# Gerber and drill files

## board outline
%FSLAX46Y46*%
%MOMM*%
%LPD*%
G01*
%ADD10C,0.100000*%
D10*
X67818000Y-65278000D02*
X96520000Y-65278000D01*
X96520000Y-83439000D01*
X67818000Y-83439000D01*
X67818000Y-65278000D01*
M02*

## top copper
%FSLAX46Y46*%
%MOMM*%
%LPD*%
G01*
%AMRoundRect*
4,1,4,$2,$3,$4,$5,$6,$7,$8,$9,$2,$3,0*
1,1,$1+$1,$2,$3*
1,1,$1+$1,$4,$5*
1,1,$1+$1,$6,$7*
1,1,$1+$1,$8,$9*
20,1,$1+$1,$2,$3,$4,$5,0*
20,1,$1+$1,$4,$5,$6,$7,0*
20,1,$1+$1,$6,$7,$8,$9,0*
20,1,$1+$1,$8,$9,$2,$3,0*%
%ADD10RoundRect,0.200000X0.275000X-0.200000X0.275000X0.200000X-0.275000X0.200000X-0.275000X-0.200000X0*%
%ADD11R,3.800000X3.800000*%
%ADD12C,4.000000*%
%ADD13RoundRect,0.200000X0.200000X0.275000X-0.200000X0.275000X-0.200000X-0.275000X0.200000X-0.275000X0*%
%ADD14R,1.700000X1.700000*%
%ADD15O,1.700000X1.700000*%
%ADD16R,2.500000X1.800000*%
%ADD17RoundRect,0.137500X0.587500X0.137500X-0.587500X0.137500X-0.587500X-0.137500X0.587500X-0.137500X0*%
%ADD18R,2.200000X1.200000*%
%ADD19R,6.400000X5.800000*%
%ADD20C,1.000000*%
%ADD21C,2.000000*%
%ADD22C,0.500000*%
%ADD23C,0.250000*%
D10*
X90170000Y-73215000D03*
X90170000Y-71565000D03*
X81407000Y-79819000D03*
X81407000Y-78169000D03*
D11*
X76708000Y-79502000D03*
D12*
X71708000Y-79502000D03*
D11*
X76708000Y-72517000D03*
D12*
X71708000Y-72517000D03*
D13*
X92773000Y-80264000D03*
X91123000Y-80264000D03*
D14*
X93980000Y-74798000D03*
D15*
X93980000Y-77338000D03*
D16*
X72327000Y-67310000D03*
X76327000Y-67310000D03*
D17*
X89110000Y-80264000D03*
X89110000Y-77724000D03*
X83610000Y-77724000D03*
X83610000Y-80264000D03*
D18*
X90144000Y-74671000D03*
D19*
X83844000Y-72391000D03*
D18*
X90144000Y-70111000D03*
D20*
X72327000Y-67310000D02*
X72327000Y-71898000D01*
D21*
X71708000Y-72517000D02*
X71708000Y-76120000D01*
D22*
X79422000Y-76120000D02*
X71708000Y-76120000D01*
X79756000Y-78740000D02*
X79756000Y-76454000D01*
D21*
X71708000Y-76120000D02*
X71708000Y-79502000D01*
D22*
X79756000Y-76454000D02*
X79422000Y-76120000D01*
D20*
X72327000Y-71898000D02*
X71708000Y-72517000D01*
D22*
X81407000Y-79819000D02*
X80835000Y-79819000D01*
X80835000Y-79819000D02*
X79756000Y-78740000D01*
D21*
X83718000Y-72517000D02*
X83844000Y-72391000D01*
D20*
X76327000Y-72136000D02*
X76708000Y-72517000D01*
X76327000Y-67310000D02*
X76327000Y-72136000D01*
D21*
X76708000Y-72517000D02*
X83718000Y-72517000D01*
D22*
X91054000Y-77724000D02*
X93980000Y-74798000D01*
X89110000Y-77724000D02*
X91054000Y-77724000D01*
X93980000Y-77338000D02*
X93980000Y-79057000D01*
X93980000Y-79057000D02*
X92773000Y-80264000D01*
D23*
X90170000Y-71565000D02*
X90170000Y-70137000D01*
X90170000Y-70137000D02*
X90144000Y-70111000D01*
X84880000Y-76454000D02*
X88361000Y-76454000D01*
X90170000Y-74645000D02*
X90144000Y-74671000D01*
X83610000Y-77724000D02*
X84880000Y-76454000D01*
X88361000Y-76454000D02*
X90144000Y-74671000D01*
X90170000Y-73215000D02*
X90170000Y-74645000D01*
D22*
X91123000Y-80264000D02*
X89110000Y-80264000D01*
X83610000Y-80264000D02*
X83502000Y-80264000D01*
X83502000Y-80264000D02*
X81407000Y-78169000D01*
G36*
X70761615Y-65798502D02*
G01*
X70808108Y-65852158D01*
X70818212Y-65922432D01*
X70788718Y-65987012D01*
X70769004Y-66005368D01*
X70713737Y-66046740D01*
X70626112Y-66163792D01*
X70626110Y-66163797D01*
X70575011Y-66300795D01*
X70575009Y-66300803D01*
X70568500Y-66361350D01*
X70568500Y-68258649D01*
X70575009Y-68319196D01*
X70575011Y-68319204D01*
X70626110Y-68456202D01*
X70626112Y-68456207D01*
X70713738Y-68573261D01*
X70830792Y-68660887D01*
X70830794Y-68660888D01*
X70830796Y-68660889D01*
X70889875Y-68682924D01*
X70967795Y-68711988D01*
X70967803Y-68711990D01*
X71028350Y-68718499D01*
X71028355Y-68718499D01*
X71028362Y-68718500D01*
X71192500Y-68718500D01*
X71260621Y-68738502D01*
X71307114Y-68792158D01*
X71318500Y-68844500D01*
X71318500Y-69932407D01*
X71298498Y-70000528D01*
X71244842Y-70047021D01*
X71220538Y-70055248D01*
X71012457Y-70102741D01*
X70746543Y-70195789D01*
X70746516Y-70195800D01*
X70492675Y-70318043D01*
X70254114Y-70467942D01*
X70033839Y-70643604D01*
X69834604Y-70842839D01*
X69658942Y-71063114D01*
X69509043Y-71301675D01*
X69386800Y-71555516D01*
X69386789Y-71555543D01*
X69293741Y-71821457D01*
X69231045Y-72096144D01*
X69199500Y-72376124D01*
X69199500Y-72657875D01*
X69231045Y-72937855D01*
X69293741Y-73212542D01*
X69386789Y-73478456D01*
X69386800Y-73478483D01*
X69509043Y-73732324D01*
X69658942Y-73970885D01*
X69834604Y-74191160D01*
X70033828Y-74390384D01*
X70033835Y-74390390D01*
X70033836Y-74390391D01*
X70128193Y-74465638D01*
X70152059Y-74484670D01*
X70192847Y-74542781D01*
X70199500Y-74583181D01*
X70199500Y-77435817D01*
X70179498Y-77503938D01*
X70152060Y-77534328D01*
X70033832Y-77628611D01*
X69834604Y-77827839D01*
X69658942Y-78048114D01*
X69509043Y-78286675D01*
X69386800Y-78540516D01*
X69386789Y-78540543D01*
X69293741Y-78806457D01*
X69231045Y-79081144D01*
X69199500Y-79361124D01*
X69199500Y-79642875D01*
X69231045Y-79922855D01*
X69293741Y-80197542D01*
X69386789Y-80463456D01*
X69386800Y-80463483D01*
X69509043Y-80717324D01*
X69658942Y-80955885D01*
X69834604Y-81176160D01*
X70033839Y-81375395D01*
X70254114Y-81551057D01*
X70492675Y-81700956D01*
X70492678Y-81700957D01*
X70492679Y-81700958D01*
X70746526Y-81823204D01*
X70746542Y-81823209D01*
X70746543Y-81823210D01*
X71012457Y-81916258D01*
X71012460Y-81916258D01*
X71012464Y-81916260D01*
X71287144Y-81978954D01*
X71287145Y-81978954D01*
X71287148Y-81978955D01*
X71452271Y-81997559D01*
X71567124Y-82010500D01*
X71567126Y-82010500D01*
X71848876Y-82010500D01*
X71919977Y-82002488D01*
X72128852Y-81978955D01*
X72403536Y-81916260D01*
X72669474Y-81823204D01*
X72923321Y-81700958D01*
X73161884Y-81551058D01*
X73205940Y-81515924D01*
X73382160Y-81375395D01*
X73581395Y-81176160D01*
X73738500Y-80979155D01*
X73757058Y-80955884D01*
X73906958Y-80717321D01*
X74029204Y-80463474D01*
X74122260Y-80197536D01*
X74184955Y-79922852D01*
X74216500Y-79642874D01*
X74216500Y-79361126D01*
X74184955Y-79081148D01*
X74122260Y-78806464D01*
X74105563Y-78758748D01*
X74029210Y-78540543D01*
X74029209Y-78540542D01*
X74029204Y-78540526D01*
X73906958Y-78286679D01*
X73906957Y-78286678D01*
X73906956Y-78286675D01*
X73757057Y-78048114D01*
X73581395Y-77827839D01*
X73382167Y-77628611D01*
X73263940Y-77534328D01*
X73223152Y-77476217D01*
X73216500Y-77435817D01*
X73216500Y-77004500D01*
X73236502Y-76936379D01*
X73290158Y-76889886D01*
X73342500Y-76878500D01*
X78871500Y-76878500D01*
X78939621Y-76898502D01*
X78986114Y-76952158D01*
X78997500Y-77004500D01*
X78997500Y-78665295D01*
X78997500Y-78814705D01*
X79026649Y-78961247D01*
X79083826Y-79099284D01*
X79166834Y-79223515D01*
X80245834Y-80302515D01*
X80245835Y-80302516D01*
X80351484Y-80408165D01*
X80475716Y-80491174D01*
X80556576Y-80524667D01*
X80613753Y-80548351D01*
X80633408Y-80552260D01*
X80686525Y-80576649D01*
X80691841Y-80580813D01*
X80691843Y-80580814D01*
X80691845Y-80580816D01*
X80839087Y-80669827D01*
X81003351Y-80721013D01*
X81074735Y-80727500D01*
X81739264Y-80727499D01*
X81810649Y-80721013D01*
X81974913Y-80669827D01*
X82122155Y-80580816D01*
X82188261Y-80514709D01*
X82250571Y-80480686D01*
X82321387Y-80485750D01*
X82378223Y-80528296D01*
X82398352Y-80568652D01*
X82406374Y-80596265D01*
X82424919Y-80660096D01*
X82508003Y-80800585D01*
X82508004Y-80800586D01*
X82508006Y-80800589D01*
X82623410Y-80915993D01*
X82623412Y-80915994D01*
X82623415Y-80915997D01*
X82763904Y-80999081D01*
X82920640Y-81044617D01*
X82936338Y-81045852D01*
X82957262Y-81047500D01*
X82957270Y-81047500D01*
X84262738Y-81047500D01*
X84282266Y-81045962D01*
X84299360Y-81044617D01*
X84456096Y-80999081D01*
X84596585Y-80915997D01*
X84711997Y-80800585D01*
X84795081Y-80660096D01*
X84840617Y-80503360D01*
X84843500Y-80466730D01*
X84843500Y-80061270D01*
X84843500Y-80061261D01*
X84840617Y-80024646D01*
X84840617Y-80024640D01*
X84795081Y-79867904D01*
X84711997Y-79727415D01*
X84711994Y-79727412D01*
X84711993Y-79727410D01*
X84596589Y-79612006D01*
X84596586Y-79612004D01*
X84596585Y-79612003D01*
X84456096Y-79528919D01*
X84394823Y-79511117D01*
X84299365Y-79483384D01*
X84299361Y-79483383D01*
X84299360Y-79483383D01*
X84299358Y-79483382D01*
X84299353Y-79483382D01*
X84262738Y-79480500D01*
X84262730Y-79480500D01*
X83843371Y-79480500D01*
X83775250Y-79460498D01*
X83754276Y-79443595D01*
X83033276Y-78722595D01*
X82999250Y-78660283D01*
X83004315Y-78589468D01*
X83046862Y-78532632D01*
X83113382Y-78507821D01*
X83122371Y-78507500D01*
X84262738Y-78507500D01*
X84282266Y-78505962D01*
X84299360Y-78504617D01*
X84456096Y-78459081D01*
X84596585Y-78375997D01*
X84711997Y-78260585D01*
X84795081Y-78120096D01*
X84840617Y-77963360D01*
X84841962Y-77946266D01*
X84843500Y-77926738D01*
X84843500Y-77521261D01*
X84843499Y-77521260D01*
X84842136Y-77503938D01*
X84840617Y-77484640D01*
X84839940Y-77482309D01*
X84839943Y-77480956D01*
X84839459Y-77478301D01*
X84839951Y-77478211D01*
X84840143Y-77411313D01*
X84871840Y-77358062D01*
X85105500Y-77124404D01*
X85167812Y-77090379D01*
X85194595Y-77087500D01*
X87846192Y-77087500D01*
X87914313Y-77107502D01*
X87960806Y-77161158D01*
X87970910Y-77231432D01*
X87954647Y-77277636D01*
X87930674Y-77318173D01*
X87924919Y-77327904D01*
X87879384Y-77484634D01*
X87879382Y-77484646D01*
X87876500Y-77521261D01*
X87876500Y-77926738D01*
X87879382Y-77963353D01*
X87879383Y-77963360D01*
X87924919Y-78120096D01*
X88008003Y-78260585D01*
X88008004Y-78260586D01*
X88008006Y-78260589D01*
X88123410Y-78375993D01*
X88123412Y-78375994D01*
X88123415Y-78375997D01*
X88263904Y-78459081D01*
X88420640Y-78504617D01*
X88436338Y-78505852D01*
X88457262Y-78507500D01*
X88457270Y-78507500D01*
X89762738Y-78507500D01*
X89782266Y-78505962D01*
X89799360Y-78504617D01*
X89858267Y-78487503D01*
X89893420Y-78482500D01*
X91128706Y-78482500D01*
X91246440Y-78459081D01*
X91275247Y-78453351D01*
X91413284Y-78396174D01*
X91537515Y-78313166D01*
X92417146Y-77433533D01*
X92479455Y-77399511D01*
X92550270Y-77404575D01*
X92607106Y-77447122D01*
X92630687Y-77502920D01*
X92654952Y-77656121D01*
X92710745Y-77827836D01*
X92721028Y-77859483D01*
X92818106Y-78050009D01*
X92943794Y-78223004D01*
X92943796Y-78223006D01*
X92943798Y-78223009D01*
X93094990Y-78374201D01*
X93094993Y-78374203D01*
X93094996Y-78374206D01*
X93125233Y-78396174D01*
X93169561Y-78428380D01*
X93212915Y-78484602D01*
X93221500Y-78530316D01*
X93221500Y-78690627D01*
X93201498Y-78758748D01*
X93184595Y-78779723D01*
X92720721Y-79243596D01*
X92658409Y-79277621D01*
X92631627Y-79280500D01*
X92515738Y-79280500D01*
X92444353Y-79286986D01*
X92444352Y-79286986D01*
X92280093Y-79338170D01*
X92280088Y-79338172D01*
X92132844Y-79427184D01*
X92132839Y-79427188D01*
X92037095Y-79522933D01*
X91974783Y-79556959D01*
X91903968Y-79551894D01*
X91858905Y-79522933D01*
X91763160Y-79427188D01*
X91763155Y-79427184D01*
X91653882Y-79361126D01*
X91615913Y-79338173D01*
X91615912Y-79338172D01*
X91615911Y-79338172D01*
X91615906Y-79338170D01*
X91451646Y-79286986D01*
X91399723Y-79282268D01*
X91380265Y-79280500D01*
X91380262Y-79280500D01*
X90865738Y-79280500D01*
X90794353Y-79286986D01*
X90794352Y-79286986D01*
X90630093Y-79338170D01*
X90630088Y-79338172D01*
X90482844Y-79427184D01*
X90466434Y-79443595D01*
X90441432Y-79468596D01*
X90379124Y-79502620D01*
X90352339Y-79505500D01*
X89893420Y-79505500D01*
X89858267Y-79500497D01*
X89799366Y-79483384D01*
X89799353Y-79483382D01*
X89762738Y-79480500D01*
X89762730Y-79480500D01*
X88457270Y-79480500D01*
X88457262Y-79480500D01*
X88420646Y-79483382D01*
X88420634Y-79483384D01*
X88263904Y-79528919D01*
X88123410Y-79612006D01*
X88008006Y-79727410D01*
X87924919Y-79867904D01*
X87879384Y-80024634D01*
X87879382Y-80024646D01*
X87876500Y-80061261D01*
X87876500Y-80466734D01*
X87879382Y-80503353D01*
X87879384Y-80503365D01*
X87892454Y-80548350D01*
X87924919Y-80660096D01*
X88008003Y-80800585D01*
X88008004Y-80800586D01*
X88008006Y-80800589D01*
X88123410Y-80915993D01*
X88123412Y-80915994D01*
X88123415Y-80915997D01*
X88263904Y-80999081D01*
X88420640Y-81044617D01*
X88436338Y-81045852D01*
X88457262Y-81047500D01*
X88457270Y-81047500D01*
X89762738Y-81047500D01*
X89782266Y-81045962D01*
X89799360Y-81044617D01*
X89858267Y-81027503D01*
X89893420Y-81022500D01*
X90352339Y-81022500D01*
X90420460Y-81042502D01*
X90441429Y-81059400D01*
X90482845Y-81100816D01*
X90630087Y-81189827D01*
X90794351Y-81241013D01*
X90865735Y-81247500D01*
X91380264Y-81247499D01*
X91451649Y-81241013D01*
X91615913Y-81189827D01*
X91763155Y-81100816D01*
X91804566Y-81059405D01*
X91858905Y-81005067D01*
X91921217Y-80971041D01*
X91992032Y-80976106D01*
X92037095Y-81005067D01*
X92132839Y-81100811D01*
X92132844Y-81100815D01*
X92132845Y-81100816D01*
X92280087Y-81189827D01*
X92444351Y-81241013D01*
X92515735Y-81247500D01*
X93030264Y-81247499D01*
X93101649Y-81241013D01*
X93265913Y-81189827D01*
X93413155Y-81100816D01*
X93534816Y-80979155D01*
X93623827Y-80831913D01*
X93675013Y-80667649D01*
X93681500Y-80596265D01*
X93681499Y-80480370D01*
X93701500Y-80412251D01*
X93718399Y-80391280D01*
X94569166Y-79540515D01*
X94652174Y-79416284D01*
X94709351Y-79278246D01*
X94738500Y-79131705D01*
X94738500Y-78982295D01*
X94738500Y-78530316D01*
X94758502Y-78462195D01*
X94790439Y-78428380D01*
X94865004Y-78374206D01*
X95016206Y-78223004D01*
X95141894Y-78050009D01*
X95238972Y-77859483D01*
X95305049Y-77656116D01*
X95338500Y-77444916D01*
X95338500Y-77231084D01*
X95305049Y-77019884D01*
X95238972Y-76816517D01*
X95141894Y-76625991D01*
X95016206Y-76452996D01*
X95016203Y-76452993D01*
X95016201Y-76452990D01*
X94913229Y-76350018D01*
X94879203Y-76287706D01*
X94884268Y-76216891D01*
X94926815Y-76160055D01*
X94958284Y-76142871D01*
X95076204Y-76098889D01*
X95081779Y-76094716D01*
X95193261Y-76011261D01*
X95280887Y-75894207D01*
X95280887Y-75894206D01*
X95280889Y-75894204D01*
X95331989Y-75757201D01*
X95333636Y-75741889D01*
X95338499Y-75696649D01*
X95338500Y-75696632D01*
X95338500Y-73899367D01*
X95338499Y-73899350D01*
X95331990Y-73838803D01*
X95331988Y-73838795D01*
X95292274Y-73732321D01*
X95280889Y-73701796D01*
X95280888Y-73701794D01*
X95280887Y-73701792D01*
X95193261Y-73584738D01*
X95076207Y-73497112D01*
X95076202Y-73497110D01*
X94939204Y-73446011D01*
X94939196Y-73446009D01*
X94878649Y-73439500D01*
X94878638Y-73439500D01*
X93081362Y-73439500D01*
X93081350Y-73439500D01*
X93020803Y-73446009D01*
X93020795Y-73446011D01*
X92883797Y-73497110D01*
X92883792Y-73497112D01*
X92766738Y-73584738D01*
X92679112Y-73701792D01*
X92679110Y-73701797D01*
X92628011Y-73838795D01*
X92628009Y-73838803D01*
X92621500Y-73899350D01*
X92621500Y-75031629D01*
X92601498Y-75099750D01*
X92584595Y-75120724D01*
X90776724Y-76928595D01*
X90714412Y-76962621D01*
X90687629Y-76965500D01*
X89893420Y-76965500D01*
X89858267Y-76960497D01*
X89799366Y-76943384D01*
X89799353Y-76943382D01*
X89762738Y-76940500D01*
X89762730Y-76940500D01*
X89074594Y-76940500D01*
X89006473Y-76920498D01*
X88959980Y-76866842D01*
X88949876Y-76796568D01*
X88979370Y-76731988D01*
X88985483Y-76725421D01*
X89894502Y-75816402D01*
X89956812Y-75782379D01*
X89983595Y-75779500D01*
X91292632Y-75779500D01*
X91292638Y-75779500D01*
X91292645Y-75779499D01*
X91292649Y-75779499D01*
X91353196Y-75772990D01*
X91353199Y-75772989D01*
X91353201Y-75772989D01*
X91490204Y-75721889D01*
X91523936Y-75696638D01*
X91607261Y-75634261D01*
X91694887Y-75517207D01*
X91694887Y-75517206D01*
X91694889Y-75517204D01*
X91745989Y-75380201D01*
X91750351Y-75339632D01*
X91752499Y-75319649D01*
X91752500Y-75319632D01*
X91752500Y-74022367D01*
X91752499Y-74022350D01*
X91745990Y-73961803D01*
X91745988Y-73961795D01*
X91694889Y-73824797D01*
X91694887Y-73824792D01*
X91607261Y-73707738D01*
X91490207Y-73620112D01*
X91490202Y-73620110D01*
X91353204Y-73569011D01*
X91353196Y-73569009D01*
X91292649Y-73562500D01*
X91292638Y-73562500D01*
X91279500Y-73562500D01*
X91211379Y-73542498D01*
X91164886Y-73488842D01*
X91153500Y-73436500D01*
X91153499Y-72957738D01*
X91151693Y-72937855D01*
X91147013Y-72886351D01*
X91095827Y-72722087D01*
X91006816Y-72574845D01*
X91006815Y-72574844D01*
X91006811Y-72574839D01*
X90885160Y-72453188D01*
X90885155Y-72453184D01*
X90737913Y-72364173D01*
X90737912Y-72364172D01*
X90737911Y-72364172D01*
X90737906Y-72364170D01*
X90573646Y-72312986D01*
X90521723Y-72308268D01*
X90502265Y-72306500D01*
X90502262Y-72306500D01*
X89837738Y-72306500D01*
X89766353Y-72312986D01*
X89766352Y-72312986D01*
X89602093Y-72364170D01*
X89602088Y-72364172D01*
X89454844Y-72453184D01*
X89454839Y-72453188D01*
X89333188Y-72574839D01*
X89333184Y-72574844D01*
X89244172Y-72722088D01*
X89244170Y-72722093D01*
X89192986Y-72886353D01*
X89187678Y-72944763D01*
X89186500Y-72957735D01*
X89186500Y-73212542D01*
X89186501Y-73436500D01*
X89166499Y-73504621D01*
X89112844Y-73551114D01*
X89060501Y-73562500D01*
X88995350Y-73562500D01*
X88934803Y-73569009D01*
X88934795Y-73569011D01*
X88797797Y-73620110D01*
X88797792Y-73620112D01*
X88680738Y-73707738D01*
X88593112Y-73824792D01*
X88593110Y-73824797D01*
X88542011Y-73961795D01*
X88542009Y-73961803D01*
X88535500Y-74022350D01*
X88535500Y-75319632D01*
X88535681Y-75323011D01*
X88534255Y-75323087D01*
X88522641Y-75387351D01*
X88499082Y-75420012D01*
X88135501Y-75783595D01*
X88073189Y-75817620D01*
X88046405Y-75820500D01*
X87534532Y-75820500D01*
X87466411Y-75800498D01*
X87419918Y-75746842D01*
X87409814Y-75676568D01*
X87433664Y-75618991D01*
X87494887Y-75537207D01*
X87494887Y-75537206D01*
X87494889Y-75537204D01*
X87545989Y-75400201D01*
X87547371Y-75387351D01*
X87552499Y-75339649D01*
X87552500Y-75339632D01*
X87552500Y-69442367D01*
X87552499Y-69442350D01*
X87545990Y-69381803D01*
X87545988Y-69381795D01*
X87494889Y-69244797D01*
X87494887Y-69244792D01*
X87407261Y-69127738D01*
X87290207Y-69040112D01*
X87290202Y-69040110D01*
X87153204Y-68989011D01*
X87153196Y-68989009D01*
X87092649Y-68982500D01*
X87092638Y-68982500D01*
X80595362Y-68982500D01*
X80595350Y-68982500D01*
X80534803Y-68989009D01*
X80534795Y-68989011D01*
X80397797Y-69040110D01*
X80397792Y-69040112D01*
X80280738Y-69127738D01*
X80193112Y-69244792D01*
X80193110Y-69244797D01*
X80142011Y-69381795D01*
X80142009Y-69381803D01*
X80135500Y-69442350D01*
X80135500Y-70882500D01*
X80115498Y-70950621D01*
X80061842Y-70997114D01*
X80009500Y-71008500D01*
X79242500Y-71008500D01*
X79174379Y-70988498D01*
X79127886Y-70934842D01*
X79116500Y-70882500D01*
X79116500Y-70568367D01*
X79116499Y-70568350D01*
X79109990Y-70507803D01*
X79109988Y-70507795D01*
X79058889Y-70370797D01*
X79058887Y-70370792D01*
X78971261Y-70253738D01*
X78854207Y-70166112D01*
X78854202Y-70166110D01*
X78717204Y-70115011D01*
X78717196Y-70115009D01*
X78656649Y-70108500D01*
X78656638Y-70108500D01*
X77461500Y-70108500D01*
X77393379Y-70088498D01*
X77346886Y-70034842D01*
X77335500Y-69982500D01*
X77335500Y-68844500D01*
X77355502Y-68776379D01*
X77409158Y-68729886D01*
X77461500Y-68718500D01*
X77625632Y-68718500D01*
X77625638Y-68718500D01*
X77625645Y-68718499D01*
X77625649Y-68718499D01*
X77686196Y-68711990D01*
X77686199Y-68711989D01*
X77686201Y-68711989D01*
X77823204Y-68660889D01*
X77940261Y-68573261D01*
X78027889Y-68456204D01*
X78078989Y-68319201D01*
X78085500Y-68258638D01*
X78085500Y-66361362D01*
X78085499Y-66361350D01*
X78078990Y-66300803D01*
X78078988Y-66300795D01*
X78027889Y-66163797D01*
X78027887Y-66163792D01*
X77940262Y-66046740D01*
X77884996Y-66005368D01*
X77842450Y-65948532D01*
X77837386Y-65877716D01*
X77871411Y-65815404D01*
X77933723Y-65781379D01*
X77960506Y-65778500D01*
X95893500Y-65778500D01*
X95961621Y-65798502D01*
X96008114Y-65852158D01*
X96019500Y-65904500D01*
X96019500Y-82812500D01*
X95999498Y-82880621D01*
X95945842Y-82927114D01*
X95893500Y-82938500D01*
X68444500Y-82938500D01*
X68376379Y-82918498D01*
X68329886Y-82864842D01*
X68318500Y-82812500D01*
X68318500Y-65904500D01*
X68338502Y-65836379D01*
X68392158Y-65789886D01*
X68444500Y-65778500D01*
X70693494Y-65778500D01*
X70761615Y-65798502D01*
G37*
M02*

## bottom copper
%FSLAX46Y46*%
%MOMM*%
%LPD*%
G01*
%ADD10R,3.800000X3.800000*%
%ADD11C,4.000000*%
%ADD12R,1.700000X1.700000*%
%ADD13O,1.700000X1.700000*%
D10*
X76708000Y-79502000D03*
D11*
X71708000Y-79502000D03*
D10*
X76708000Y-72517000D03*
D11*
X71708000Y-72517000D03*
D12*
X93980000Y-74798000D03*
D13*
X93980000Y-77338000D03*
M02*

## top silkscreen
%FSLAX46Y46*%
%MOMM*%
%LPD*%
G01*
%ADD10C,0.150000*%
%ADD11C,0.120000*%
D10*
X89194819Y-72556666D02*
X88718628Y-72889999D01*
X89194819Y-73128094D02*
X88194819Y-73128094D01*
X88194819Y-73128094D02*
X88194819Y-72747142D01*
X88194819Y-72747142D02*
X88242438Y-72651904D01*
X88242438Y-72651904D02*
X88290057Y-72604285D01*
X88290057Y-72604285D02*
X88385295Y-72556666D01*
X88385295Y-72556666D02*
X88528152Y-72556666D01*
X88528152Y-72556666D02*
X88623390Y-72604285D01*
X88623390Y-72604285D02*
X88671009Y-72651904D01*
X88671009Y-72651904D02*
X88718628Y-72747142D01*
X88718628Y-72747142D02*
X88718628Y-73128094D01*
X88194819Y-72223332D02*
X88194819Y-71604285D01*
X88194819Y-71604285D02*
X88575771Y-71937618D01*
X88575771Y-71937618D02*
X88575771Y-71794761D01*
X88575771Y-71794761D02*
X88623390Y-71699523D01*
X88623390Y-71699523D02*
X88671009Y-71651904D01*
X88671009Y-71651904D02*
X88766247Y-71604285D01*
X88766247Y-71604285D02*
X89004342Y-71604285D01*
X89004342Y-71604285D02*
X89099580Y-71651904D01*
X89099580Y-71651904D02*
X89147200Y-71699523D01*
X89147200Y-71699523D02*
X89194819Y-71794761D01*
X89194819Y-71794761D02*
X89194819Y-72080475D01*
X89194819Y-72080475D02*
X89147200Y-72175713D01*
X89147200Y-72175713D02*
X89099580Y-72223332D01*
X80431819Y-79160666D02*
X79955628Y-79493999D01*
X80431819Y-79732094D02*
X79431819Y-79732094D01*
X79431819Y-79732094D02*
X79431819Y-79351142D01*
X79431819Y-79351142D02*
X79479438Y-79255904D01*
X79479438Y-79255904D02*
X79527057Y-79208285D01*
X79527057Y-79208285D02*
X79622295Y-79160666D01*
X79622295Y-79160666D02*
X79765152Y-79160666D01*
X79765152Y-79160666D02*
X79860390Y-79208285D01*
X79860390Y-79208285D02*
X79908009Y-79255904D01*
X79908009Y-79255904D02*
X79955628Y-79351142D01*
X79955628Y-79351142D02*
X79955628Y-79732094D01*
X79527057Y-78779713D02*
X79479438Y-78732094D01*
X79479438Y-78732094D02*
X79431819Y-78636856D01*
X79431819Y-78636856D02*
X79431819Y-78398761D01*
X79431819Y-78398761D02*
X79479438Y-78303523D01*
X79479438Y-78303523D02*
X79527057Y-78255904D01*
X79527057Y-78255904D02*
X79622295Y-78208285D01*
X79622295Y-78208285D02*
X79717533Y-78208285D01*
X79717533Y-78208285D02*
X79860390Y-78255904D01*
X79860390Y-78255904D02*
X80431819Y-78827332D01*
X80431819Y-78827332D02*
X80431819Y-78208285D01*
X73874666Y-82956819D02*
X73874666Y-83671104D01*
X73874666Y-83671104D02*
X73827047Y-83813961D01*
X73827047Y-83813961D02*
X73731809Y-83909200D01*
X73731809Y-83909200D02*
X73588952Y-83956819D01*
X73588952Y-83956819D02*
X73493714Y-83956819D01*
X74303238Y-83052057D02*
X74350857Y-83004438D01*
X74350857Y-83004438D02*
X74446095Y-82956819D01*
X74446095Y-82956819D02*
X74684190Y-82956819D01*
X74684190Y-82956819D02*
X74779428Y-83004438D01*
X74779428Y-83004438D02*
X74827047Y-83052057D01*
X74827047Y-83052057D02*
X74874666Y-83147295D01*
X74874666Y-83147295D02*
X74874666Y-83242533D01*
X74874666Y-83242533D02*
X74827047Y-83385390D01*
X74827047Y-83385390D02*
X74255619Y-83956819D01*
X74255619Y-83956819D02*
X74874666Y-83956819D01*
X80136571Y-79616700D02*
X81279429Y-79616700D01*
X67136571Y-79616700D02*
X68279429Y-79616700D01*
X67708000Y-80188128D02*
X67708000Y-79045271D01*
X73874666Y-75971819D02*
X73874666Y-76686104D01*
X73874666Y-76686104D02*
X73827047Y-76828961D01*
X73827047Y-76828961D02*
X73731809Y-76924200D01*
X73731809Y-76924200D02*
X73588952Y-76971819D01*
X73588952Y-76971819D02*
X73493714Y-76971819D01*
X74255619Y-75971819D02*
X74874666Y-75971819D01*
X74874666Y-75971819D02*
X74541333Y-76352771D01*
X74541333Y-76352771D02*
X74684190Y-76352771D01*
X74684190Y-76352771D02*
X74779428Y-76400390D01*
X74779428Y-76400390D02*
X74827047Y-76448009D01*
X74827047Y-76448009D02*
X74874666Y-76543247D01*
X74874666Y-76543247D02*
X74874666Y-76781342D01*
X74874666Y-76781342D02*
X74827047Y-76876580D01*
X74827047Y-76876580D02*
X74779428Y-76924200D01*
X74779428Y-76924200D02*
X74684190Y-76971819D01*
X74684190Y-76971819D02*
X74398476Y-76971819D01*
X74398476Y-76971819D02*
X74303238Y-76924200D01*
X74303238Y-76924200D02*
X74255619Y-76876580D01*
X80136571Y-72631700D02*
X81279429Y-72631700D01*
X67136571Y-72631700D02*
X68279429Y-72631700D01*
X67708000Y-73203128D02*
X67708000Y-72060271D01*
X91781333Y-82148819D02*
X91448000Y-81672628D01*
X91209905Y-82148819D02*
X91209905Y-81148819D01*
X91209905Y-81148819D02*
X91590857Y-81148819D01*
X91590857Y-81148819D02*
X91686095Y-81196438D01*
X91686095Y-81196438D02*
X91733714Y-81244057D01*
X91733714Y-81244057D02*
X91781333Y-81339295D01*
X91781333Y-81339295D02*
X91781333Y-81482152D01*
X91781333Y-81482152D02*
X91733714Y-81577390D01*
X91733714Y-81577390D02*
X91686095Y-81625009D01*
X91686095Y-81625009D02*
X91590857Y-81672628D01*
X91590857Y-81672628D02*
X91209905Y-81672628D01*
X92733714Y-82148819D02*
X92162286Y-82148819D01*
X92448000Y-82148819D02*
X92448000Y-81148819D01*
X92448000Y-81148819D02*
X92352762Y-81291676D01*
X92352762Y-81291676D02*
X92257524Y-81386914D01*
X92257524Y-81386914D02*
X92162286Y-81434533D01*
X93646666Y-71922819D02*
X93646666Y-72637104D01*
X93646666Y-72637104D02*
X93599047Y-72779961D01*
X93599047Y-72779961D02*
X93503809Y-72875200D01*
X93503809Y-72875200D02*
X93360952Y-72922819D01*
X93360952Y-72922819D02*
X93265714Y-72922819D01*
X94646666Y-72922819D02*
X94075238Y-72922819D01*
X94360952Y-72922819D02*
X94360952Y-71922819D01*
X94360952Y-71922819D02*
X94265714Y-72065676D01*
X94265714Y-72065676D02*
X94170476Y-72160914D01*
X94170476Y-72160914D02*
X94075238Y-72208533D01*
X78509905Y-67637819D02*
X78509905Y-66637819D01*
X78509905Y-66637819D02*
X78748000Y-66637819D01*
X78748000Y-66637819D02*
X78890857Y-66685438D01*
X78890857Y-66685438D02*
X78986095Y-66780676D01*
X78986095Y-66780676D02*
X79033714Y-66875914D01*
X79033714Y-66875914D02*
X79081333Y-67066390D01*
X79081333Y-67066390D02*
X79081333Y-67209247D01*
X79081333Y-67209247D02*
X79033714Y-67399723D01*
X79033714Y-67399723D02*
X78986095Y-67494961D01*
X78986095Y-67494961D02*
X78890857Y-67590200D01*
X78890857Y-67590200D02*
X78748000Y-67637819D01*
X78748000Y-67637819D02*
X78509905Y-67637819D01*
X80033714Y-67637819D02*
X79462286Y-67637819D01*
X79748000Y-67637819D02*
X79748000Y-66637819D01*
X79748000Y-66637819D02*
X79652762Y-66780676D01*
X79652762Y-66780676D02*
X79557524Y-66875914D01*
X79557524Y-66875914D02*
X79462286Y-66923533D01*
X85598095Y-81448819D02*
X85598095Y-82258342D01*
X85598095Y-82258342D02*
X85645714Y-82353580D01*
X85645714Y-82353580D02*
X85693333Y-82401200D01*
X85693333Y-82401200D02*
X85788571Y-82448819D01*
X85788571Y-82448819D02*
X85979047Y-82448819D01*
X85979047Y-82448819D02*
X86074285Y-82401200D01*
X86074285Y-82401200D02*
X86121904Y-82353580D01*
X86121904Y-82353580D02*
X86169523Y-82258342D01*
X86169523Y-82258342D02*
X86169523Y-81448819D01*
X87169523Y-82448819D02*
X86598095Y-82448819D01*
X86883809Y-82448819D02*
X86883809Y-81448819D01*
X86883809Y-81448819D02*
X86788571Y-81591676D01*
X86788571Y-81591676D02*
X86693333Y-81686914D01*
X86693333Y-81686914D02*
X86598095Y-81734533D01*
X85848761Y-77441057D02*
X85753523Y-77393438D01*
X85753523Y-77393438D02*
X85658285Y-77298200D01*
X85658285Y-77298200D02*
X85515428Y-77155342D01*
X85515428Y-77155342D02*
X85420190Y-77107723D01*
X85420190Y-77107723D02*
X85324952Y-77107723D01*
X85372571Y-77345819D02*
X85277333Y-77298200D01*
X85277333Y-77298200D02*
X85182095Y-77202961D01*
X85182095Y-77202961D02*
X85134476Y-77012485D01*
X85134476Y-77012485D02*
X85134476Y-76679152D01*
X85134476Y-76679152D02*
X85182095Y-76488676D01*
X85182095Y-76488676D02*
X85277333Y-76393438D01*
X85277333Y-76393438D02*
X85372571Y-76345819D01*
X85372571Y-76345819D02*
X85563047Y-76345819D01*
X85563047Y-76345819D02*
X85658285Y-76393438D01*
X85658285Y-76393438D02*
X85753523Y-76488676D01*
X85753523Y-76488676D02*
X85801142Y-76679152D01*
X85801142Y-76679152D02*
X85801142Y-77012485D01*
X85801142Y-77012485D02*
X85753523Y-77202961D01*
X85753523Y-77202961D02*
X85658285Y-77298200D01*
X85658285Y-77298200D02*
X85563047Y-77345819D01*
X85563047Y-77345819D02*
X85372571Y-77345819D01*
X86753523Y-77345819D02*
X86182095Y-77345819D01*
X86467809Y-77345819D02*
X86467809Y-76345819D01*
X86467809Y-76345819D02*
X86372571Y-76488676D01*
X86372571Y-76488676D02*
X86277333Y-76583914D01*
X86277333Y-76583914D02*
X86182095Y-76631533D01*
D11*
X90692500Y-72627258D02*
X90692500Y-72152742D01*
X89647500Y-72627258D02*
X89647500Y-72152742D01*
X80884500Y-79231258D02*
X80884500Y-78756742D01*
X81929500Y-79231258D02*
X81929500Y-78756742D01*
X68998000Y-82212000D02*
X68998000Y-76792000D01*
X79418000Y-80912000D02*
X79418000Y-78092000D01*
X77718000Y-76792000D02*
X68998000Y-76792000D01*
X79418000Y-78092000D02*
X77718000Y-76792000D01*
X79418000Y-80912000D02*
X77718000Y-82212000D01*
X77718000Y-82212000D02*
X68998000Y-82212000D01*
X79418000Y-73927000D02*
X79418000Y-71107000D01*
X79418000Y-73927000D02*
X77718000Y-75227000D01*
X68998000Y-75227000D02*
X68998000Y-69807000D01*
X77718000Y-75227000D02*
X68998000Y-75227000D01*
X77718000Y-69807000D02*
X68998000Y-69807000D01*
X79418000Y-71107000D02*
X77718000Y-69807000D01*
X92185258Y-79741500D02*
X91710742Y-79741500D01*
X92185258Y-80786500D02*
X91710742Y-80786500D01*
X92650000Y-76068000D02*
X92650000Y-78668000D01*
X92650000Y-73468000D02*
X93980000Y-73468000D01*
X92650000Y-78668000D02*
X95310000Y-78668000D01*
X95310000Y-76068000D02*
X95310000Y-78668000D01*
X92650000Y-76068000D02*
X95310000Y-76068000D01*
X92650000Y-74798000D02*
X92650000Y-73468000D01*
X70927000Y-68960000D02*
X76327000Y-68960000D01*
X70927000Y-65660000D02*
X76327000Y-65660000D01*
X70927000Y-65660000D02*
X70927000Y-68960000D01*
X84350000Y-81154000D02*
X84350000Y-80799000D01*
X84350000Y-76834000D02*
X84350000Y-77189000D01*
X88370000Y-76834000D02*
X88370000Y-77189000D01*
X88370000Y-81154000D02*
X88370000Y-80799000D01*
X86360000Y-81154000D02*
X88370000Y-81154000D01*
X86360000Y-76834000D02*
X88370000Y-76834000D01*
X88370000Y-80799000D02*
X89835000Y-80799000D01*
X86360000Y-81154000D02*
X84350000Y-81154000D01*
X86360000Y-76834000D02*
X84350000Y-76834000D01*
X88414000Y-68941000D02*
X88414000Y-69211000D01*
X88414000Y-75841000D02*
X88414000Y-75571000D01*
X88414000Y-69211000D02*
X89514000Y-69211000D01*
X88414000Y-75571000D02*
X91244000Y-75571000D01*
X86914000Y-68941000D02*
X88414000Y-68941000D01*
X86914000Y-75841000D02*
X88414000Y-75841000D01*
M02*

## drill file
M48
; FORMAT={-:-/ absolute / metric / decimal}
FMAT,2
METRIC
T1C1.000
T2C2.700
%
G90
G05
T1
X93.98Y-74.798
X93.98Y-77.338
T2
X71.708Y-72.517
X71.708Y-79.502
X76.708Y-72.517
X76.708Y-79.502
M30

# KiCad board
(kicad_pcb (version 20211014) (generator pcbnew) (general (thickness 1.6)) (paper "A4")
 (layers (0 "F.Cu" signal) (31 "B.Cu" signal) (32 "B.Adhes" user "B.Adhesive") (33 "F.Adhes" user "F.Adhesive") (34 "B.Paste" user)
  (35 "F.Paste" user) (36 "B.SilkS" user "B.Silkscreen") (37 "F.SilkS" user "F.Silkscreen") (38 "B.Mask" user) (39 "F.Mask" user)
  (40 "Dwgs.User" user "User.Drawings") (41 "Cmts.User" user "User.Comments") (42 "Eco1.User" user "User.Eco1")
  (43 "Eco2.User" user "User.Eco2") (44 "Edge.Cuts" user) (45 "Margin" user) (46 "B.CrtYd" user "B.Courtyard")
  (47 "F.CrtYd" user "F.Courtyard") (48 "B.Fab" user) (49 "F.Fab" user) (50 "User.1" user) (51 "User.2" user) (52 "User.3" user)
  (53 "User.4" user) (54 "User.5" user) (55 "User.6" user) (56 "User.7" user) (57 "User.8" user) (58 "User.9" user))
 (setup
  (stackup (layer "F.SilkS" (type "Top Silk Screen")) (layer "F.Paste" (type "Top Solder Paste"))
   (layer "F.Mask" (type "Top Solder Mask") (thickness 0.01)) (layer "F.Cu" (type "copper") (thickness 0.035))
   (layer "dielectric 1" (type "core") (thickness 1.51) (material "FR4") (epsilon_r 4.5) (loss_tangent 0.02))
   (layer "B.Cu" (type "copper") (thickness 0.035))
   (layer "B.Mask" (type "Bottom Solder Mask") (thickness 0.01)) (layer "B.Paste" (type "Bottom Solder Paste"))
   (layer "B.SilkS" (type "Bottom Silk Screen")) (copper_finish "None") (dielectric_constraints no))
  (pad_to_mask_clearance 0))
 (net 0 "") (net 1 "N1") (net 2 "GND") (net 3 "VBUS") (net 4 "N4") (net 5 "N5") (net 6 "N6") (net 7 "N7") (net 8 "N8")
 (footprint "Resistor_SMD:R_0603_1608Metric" (layer "F.Cu") (at 90.17 72.39 90)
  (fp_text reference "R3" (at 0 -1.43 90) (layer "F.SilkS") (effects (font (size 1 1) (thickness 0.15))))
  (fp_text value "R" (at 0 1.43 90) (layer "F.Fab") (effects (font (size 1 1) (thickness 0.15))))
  (fp_line (start -0.237258 0.5225) (end 0.237258 0.5225) (layer "F.SilkS") (width 0.12))
  (fp_line (start -0.237258 -0.5225) (end 0.237258 -0.5225) (layer "F.SilkS") (width 0.12))
  (pad "1" smd roundrect (at -0.825 0 90) (size 0.8 0.95) (layers "F.Cu" "F.Paste" "F.Mask") (roundrect_rratio 0.25) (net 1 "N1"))
  (pad "2" smd roundrect (at 0.825 0 90) (size 0.8 0.95) (layers "F.Cu" "F.Paste" "F.Mask") (roundrect_rratio 0.25) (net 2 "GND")))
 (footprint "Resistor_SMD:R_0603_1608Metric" (layer "F.Cu") (at 81.407 78.994 90)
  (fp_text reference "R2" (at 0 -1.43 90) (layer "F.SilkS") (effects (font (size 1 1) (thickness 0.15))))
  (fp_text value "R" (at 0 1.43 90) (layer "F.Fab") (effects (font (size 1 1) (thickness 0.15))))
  (fp_line (start -0.237258 -0.5225) (end 0.237258 -0.5225) (layer "F.SilkS") (width 0.12))
  (fp_line (start -0.237258 0.5225) (end 0.237258 0.5225) (layer "F.SilkS") (width 0.12))
  (pad "1" smd roundrect (at -0.825 0 90) (size 0.8 0.95) (layers "F.Cu" "F.Paste" "F.Mask") (roundrect_rratio 0.25) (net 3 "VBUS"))
  (pad "2" smd roundrect (at 0.825 0 90) (size 0.8 0.95) (layers "F.Cu" "F.Paste" "F.Mask") (roundrect_rratio 0.25) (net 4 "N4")))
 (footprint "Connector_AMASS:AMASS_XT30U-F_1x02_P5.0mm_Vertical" (layer "F.Cu") (at 76.708 79.502 180)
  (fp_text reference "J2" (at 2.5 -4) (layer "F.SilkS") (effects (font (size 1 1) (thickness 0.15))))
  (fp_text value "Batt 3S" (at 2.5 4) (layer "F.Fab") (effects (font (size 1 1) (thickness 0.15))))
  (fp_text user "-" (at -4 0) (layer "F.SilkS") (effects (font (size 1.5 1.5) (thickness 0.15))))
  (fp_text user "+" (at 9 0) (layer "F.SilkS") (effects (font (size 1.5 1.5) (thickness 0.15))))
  (fp_line (start 7.71 -2.71) (end 7.71 2.71) (layer "F.SilkS") (width 0.12))
  (fp_line (start -2.71 -1.41) (end -2.71 1.41) (layer "F.SilkS") (width 0.12))
  (fp_line (start -1.01 2.71) (end 7.71 2.71) (layer "F.SilkS") (width 0.12))
  (fp_line (start -2.71 1.41) (end -1.01 2.71) (layer "F.SilkS") (width 0.12))
  (fp_line (start -2.71 -1.41) (end -1.01 -2.71) (layer "F.SilkS") (width 0.12))
  (fp_line (start -1.01 -2.71) (end 7.71 -2.71) (layer "F.SilkS") (width 0.12))
  (pad "1" thru_hole rect (at 0 0 180) (size 3.8 3.8) (drill 2.7) (layers *.Cu *.Mask) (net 2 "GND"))
  (pad "2" thru_hole circle (at 5 0 180) (size 4 4) (drill 2.7) (layers *.Cu *.Mask) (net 3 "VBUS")))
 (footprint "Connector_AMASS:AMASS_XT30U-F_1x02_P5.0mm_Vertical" (layer "F.Cu") (at 76.708 72.517 180)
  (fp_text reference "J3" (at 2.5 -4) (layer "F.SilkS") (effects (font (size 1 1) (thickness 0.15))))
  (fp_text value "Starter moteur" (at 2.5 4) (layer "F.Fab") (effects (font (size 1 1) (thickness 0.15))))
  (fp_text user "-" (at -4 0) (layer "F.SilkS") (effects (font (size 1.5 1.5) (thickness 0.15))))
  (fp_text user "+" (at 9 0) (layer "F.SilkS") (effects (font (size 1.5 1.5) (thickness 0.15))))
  (fp_line (start -2.71 -1.41) (end -2.71 1.41) (layer "F.SilkS") (width 0.12))
  (fp_line (start -2.71 -1.41) (end -1.01 -2.71) (layer "F.SilkS") (width 0.12))
  (fp_line (start 7.71 -2.71) (end 7.71 2.71) (layer "F.SilkS") (width 0.12))
  (fp_line (start -1.01 -2.71) (end 7.71 -2.71) (layer "F.SilkS") (width 0.12))
  (fp_line (start -1.01 2.71) (end 7.71 2.71) (layer "F.SilkS") (width 0.12))
  (fp_line (start -2.71 1.41) (end -1.01 2.71) (layer "F.SilkS") (width 0.12))
  (pad "1" thru_hole rect (at 0 0 180) (size 3.8 3.8) (drill 2.7) (layers *.Cu *.Mask) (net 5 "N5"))
  (pad "2" thru_hole circle (at 5 0 180) (size 4 4) (drill 2.7) (layers *.Cu *.Mask) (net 3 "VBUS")))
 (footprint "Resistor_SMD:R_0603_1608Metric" (layer "F.Cu") (at 91.948 80.264 180)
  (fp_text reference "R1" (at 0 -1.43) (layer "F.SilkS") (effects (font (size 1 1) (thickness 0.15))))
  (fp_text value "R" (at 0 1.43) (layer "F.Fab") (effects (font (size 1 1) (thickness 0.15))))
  (fp_line (start -0.237258 0.5225) (end 0.237258 0.5225) (layer "F.SilkS") (width 0.12))
  (fp_line (start -0.237258 -0.5225) (end 0.237258 -0.5225) (layer "F.SilkS") (width 0.12))
  (pad "1" smd roundrect (at -0.825 0 180) (size 0.8 0.95) (layers "F.Cu" "F.Paste" "F.Mask") (roundrect_rratio 0.25) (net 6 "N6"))
  (pad "2" smd roundrect (at 0.825 0 180) (size 0.8 0.95) (layers "F.Cu" "F.Paste" "F.Mask") (roundrect_rratio 0.25) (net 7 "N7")))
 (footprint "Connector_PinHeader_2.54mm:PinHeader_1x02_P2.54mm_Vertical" (layer "F.Cu") (at 93.98 74.798)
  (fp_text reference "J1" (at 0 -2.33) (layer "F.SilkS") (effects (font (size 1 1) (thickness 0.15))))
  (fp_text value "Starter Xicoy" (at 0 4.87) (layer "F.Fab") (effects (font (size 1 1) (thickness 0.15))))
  (fp_line (start -1.33 1.27) (end -1.33 3.87) (layer "F.SilkS") (width 0.12))
  (fp_line (start -1.33 -1.33) (end 0 -1.33) (layer "F.SilkS") (width 0.12))
  (fp_line (start -1.33 3.87) (end 1.33 3.87) (layer "F.SilkS") (width 0.12))
  (fp_line (start 1.33 1.27) (end 1.33 3.87) (layer "F.SilkS") (width 0.12))
  (fp_line (start -1.33 1.27) (end 1.33 1.27) (layer "F.SilkS") (width 0.12))
  (fp_line (start -1.33 0) (end -1.33 -1.33) (layer "F.SilkS") (width 0.12))
  (pad "1" thru_hole rect (at 0 0) (size 1.7 1.7) (drill 1) (layers *.Cu *.Mask) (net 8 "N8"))
  (pad "2" thru_hole oval (at 0 2.54) (size 1.7 1.7) (drill 1) (layers *.Cu *.Mask) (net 6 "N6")))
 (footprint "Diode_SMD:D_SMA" (layer "F.Cu") (at 74.327 67.31)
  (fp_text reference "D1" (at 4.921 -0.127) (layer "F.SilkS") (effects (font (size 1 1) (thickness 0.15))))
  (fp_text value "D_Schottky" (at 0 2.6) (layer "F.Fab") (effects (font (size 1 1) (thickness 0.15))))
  (fp_line (start -3.4 1.65) (end 2 1.65) (layer "F.SilkS") (width 0.12))
  (fp_line (start -3.4 -1.65) (end 2 -1.65) (layer "F.SilkS") (width 0.12))
  (fp_line (start -3.4 -1.65) (end -3.4 1.65) (layer "F.SilkS") (width 0.12))
  (pad "1" smd rect (at -2 0) (size 2.5 1.8) (layers "F.Cu" "F.Paste" "F.Mask") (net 3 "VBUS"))
  (pad "2" smd rect (at 2 0) (size 2.5 1.8) (layers "F.Cu" "F.Paste" "F.Mask") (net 5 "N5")))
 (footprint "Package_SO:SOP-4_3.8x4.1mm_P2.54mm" (layer "F.Cu") (at 86.36 78.994 180)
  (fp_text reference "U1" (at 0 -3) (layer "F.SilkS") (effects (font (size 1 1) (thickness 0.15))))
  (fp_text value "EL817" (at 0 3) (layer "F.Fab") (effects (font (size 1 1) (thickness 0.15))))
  (fp_line (start 2.01 -2.16) (end 2.01 -1.805) (layer "F.SilkS") (width 0.12))
  (fp_line (start 2.01 2.16) (end 2.01 1.805) (layer "F.SilkS") (width 0.12))
  (fp_line (start -2.01 2.16) (end -2.01 1.805) (layer "F.SilkS") (width 0.12))
  (fp_line (start -2.01 -2.16) (end -2.01 -1.805) (layer "F.SilkS") (width 0.12))
  (fp_line (start 0 -2.16) (end -2.01 -2.16) (layer "F.SilkS") (width 0.12))
  (fp_line (start 0 2.16) (end -2.01 2.16) (layer "F.SilkS") (width 0.12))
  (fp_line (start -2.01 -1.805) (end -3.475 -1.805) (layer "F.SilkS") (width 0.12))
  (fp_line (start 0 -2.16) (end 2.01 -2.16) (layer "F.SilkS") (width 0.12))
  (fp_line (start 0 2.16) (end 2.01 2.16) (layer "F.SilkS") (width 0.12))
  (pad "1" smd roundrect (at -2.75 -1.27 180) (size 1.45 0.55) (layers "F.Cu" "F.Paste" "F.Mask") (roundrect_rratio 0.25) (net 7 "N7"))
  (pad "2" smd roundrect (at -2.75 1.27 180) (size 1.45 0.55) (layers "F.Cu" "F.Paste" "F.Mask") (roundrect_rratio 0.25) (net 8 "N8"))
  (pad "3" smd roundrect (at 2.75 1.27 180) (size 1.45 0.55) (layers "F.Cu" "F.Paste" "F.Mask") (roundrect_rratio 0.25) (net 1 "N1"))
  (pad "4" smd roundrect (at 2.75 -1.27 180) (size 1.45 0.55) (layers "F.Cu" "F.Paste" "F.Mask") (roundrect_rratio 0.25) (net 4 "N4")))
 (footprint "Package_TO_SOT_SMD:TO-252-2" (layer "F.Cu") (at 85.944 72.391 180)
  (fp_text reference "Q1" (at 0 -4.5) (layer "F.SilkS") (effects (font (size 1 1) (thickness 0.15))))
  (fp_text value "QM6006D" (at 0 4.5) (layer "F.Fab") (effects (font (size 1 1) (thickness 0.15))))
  (fp_line (start -2.47 3.45) (end -2.47 3.18) (layer "F.SilkS") (width 0.12))
  (fp_line (start -2.47 -3.45) (end -2.47 -3.18) (layer "F.SilkS") (width 0.12))
  (fp_line (start -2.47 3.18) (end -3.57 3.18) (layer "F.SilkS") (width 0.12))
  (fp_line (start -2.47 -3.18) (end -5.3 -3.18) (layer "F.SilkS") (width 0.12))
  (fp_line (start -0.97 3.45) (end -2.47 3.45) (layer "F.SilkS") (width 0.12))
  (fp_line (start -0.97 -3.45) (end -2.47 -3.45) (layer "F.SilkS") (width 0.12))
  (pad "" smd rect (at 3.775 -1.525 180) (size 3.05 2.75) (layers "F.Paste"))
  (pad "" smd rect (at 0.425 1.525 180) (size 3.05 2.75) (layers "F.Paste"))
  (pad "" smd rect (at 3.775 1.525 180) (size 3.05 2.75) (layers "F.Paste"))
  (pad "" smd rect (at 0.425 -1.525 180) (size 3.05 2.75) (layers "F.Paste"))
  (pad "1" smd rect (at -4.2 -2.28 180) (size 2.2 1.2) (layers "F.Cu" "F.Paste" "F.Mask") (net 1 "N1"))
  (pad "2" smd rect (at 2.1 0 180) (size 6.4 5.8) (layers "F.Cu" "F.Mask") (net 5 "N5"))
  (pad "3" smd rect (at -4.2 2.28 180) (size 2.2 1.2) (layers "F.Cu" "F.Paste" "F.Mask") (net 2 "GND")))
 (gr_rect (start 67.818 65.278) (end 96.52 83.439) (layer "Edge.Cuts") (width 0.1) (fill none))
 (segment (start 72.327 67.31) (end 72.327 71.898) (width 1) (layer "F.Cu") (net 3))
 (segment (start 71.708 72.517) (end 71.708 76.12) (width 2) (layer "F.Cu") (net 3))
 (segment (start 79.422 76.12) (end 71.708 76.12) (width 0.5) (layer "F.Cu") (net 3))
 (segment (start 79.756 78.74) (end 79.756 76.454) (width 0.5) (layer "F.Cu") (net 3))
 (segment (start 71.708 76.12) (end 71.708 79.502) (width 2) (layer "F.Cu") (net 3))
 (segment (start 79.756 76.454) (end 79.422 76.12) (width 0.5) (layer "F.Cu") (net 3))
 (segment (start 72.327 71.898) (end 71.708 72.517) (width 1) (layer "F.Cu") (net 3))
 (segment (start 81.407 79.819) (end 80.835 79.819) (width 0.5) (layer "F.Cu") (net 3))
 (segment (start 80.835 79.819) (end 79.756 78.74) (width 0.5) (layer "F.Cu") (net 3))
 (segment (start 83.718 72.517) (end 83.844 72.391) (width 2) (layer "F.Cu") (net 5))
 (segment (start 76.327 72.136) (end 76.708 72.517) (width 1) (layer "F.Cu") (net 5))
 (segment (start 76.327 67.31) (end 76.327 72.136) (width 1) (layer "F.Cu") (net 5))
 (segment (start 76.708 72.517) (end 83.718 72.517) (width 2) (layer "F.Cu") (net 5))
 (segment (start 91.054 77.724) (end 93.98 74.798) (width 0.5) (layer "F.Cu") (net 8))
 (segment (start 89.11 77.724) (end 91.054 77.724) (width 0.5) (layer "F.Cu") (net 8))
 (segment (start 93.98 77.338) (end 93.98 79.057) (width 0.5) (layer "F.Cu") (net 6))
 (segment (start 93.98 79.057) (end 92.773 80.264) (width 0.5) (layer "F.Cu") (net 6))
 (segment (start 90.17 71.565) (end 90.17 70.137) (width 0.25) (layer "F.Cu") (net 2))
 (segment (start 90.17 70.137) (end 90.144 70.111) (width 0.25) (layer "F.Cu") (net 2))
 (segment (start 84.88 76.454) (end 88.361 76.454) (width 0.25) (layer "F.Cu") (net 1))
 (segment (start 90.17 74.645) (end 90.144 74.671) (width 0.25) (layer "F.Cu") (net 1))
 (segment (start 83.61 77.724) (end 84.88 76.454) (width 0.25) (layer "F.Cu") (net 1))
 (segment (start 88.361 76.454) (end 90.144 74.671) (width 0.25) (layer "F.Cu") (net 1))
 (segment (start 90.17 73.215) (end 90.17 74.645) (width 0.25) (layer "F.Cu") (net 1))
 (segment (start 91.123 80.264) (end 89.11 80.264) (width 0.5) (layer "F.Cu") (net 7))
 (segment (start 83.61 80.264) (end 83.502 80.264) (width 0.5) (layer "F.Cu") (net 4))
 (segment (start 83.502 80.264) (end 81.407 78.169) (width 0.5) (layer "F.Cu") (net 4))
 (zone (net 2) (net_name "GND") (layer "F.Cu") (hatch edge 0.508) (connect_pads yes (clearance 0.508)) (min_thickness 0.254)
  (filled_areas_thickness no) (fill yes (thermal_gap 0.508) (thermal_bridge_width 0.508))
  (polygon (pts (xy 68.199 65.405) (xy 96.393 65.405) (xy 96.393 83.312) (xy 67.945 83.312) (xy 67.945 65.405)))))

